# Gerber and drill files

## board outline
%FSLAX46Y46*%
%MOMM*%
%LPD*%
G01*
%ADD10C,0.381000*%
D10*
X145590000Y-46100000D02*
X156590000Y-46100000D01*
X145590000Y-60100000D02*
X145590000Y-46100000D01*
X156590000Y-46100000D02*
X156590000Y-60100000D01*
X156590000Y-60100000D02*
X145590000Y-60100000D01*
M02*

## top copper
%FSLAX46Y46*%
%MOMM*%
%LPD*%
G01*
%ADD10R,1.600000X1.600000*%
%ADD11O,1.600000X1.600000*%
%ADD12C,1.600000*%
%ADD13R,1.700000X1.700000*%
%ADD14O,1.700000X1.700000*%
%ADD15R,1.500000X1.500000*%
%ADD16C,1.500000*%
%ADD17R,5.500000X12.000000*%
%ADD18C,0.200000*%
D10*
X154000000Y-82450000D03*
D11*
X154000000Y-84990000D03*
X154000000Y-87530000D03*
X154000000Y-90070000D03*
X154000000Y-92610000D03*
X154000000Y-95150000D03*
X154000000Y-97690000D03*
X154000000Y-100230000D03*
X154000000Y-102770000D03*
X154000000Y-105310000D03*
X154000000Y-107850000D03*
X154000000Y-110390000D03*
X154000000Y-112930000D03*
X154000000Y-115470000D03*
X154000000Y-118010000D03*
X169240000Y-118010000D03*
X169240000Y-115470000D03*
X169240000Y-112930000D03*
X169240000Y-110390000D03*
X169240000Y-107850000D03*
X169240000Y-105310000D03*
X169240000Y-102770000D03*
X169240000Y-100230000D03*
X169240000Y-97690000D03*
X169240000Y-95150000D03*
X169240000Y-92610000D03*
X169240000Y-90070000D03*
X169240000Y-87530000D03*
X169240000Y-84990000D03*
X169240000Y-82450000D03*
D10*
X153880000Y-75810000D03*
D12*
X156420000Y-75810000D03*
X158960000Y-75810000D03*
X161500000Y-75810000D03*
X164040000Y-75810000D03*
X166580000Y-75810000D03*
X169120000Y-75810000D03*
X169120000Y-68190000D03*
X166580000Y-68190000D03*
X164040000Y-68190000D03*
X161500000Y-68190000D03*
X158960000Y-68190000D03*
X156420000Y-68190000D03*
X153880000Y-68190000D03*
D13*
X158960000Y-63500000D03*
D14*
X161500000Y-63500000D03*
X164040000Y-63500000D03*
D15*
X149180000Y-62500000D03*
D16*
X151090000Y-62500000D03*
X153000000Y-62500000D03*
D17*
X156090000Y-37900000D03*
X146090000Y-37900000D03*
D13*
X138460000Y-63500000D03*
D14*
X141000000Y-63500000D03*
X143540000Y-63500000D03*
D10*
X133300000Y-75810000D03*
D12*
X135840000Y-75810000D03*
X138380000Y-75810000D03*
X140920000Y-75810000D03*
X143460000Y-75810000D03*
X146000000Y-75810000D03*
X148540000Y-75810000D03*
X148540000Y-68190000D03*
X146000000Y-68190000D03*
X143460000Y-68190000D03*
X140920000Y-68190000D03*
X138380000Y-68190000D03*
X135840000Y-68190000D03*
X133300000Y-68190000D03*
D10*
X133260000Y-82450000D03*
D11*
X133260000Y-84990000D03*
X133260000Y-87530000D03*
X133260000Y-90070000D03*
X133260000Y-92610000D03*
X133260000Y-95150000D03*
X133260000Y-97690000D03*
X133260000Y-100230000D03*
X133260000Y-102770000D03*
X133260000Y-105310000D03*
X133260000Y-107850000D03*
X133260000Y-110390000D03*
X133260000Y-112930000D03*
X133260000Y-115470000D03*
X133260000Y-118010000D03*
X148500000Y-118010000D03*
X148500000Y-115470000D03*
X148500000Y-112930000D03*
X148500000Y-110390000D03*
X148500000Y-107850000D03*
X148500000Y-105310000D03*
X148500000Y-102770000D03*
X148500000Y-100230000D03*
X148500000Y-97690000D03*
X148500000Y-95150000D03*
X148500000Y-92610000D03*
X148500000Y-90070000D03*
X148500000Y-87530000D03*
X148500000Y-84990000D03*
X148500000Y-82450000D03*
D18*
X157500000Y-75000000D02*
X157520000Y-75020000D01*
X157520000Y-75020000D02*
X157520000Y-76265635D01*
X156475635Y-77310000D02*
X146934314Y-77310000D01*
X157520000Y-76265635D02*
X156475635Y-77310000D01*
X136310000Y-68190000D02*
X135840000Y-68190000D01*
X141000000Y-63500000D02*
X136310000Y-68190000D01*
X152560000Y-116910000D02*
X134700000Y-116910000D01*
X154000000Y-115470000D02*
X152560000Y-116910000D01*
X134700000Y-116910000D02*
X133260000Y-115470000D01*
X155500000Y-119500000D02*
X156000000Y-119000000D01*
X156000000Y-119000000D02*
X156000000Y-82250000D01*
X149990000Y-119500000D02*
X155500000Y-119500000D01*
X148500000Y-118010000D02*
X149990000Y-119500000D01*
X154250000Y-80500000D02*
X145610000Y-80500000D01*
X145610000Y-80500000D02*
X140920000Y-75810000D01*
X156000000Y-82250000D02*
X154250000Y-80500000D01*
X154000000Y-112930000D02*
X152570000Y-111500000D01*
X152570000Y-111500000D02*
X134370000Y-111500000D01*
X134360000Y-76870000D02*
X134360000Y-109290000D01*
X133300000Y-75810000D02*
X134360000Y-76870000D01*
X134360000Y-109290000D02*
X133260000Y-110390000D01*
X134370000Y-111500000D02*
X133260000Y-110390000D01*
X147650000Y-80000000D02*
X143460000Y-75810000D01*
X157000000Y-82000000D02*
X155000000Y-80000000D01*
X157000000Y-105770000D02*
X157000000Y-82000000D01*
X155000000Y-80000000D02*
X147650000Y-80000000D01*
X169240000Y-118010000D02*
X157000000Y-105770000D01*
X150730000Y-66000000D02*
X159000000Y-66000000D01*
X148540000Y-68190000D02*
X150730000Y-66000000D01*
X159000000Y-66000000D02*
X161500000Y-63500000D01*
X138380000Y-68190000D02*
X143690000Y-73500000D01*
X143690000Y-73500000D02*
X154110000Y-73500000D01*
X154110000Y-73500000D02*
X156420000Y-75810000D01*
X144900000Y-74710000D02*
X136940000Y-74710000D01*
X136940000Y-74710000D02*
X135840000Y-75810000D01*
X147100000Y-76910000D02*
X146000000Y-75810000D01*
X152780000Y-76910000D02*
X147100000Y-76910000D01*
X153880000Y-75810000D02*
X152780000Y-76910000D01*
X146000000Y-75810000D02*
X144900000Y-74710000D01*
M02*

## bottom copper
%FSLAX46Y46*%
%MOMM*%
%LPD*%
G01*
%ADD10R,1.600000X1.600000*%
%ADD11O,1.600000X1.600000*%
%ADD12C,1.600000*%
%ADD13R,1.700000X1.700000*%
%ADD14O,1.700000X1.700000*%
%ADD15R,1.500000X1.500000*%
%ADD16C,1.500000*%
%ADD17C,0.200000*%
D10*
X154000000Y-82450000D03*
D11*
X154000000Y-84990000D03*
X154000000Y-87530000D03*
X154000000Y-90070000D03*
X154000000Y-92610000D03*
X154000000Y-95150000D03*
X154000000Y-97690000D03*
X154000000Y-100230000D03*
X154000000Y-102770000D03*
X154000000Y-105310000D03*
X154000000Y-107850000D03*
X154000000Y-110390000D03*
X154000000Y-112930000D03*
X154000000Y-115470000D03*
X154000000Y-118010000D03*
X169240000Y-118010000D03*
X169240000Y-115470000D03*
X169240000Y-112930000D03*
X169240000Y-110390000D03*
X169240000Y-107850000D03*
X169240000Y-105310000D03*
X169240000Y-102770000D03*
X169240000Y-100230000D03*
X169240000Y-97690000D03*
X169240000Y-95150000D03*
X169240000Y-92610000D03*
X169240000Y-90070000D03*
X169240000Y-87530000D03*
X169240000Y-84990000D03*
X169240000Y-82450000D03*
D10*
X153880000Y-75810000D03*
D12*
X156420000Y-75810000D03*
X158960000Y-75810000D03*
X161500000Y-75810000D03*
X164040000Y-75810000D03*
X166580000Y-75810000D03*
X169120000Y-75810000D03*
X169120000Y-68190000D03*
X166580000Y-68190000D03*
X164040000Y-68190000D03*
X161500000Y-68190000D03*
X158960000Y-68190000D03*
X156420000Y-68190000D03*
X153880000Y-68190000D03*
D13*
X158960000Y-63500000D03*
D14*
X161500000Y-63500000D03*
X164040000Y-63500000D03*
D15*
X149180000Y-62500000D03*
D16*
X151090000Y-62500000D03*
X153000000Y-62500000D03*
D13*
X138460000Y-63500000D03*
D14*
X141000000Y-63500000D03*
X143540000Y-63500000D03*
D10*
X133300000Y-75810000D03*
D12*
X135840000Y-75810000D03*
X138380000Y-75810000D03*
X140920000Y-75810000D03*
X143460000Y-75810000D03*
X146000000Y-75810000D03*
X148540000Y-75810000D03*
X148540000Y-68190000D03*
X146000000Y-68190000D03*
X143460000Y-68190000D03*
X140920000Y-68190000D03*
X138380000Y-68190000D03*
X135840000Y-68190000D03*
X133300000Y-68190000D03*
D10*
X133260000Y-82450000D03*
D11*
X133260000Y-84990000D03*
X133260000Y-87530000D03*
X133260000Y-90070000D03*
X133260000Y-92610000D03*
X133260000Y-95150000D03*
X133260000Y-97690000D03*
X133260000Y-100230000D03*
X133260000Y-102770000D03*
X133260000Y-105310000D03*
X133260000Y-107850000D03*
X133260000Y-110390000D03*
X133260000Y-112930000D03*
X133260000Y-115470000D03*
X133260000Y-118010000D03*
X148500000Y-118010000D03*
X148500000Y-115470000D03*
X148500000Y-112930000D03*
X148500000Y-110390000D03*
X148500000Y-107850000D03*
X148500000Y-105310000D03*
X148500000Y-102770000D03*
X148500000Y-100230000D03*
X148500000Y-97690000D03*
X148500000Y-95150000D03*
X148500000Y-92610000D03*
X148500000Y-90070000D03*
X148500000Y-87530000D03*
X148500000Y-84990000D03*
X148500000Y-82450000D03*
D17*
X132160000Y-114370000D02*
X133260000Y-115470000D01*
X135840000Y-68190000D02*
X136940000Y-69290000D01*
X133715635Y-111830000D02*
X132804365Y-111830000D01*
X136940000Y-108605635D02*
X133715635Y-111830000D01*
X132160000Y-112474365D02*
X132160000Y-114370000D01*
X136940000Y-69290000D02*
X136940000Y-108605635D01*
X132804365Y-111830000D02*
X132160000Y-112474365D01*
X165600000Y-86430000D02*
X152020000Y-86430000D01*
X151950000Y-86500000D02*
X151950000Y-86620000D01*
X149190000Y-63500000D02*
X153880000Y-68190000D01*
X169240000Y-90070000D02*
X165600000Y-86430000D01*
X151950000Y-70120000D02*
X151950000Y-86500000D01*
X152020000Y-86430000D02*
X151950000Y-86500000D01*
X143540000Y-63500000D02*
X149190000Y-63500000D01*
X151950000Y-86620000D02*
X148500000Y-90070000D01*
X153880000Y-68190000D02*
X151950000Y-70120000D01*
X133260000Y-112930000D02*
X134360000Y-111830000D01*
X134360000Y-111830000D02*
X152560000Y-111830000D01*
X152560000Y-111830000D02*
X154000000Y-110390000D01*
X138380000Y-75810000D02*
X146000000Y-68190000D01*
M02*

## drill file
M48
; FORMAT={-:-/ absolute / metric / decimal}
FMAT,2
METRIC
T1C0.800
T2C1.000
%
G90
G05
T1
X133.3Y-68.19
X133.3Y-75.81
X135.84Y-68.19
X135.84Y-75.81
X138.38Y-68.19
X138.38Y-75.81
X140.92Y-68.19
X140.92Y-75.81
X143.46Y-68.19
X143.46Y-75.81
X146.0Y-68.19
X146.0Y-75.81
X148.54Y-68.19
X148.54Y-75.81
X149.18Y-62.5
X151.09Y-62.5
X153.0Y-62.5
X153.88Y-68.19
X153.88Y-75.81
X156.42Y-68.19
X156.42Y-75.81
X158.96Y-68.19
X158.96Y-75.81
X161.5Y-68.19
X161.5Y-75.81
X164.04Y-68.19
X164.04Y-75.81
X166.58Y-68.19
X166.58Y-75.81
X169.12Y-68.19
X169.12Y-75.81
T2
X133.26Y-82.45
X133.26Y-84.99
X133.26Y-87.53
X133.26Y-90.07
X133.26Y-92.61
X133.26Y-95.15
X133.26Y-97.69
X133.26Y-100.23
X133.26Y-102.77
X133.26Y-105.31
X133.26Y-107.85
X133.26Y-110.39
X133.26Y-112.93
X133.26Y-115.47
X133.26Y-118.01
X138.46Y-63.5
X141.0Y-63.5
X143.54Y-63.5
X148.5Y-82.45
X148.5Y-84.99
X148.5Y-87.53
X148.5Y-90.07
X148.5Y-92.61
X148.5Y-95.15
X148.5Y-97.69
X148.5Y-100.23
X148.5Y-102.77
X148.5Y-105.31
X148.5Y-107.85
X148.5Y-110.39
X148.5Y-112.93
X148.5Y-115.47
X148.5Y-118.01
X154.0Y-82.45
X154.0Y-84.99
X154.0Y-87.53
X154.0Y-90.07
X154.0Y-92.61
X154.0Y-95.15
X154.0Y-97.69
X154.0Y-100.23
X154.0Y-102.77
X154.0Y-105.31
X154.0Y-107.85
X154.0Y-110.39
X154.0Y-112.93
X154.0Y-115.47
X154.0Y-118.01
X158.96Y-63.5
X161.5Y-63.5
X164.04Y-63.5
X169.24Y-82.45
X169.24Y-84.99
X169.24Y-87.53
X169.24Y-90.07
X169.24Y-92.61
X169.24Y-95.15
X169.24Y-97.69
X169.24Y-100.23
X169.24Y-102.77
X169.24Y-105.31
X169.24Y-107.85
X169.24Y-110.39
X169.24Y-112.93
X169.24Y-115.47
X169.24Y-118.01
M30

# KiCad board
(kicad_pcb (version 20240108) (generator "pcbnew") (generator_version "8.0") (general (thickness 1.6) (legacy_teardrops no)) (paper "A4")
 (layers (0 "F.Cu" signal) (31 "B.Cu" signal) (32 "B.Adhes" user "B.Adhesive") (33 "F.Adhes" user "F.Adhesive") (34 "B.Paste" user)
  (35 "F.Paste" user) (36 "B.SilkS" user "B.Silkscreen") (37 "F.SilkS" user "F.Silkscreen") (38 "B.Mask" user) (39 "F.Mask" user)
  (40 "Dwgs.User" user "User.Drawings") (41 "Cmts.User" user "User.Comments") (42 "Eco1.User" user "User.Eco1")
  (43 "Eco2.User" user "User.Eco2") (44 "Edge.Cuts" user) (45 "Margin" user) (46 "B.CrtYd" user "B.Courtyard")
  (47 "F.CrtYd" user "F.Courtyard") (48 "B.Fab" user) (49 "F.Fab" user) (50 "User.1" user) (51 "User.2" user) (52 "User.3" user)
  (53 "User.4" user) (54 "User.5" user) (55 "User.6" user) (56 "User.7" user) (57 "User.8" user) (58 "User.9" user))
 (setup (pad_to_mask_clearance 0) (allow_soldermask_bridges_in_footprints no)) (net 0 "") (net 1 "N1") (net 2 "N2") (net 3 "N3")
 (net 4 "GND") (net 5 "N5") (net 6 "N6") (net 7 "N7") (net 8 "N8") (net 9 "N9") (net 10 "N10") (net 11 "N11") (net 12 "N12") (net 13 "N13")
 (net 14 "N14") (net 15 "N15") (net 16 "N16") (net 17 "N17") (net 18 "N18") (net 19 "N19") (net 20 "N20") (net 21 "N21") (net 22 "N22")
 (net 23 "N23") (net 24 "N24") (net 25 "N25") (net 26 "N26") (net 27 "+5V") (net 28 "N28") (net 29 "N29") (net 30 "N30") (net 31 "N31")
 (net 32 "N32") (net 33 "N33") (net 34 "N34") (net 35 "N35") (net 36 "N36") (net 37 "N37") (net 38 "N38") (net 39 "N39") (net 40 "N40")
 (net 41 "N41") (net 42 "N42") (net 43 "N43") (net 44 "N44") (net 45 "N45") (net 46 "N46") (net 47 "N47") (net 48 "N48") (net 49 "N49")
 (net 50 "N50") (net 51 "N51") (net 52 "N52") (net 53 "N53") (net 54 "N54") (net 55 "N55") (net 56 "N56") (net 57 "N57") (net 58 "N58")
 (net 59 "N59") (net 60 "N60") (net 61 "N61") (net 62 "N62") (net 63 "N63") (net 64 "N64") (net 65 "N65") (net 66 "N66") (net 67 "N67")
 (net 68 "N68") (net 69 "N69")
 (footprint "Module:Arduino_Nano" (layer "F.Cu") (at 154 82.45)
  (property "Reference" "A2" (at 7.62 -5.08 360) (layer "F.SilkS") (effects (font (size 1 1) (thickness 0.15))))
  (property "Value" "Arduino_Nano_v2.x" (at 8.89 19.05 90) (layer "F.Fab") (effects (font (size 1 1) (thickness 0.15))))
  (pad "1" thru_hole rect (at 0 0) (size 1.6 1.6) (drill 1) (layers "*.Cu" "*.Mask") (remove_unused_layers no) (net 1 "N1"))
  (pad "2" thru_hole oval (at 0 2.54) (size 1.6 1.6) (drill 1) (layers "*.Cu" "*.Mask") (remove_unused_layers no) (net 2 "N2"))
  (pad "3" thru_hole oval (at 0 5.08) (size 1.6 1.6) (drill 1) (layers "*.Cu" "*.Mask") (remove_unused_layers no) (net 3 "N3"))
  (pad "4" thru_hole oval (at 0 7.62) (size 1.6 1.6) (drill 1) (layers "*.Cu" "*.Mask") (remove_unused_layers no) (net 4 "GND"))
  (pad "5" thru_hole oval (at 0 10.16) (size 1.6 1.6) (drill 1) (layers "*.Cu" "*.Mask") (remove_unused_layers no) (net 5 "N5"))
  (pad "6" thru_hole oval (at 0 12.7) (size 1.6 1.6) (drill 1) (layers "*.Cu" "*.Mask") (remove_unused_layers no) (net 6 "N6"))
  (pad "7" thru_hole oval (at 0 15.24) (size 1.6 1.6) (drill 1) (layers "*.Cu" "*.Mask") (remove_unused_layers no) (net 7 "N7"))
  (pad "8" thru_hole oval (at 0 17.78) (size 1.6 1.6) (drill 1) (layers "*.Cu" "*.Mask") (remove_unused_layers no) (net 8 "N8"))
  (pad "9" thru_hole oval (at 0 20.32) (size 1.6 1.6) (drill 1) (layers "*.Cu" "*.Mask") (remove_unused_layers no) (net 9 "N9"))
  (pad "10" thru_hole oval (at 0 22.86) (size 1.6 1.6) (drill 1) (layers "*.Cu" "*.Mask") (remove_unused_layers no) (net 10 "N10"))
  (pad "11" thru_hole oval (at 0 25.4) (size 1.6 1.6) (drill 1) (layers "*.Cu" "*.Mask") (remove_unused_layers no) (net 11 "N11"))
  (pad "12" thru_hole oval (at 0 27.94) (size 1.6 1.6) (drill 1) (layers "*.Cu" "*.Mask") (remove_unused_layers no) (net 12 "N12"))
  (pad "13" thru_hole oval (at 0 30.48) (size 1.6 1.6) (drill 1) (layers "*.Cu" "*.Mask") (remove_unused_layers no) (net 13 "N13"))
  (pad "14" thru_hole oval (at 0 33.02) (size 1.6 1.6) (drill 1) (layers "*.Cu" "*.Mask") (remove_unused_layers no) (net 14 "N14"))
  (pad "15" thru_hole oval (at 0 35.56) (size 1.6 1.6) (drill 1) (layers "*.Cu" "*.Mask") (remove_unused_layers no) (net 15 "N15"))
  (pad "16" thru_hole oval (at 15.24 35.56) (size 1.6 1.6) (drill 1) (layers "*.Cu" "*.Mask") (remove_unused_layers no) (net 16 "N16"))
  (pad "17" thru_hole oval (at 15.24 33.02) (size 1.6 1.6) (drill 1) (layers "*.Cu" "*.Mask") (remove_unused_layers no) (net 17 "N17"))
  (pad "18" thru_hole oval (at 15.24 30.48) (size 1.6 1.6) (drill 1) (layers "*.Cu" "*.Mask") (remove_unused_layers no) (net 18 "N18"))
  (pad "19" thru_hole oval (at 15.24 27.94) (size 1.6 1.6) (drill 1) (layers "*.Cu" "*.Mask") (remove_unused_layers no) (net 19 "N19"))
  (pad "20" thru_hole oval (at 15.24 25.4) (size 1.6 1.6) (drill 1) (layers "*.Cu" "*.Mask") (remove_unused_layers no) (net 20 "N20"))
  (pad "21" thru_hole oval (at 15.24 22.86) (size 1.6 1.6) (drill 1) (layers "*.Cu" "*.Mask") (remove_unused_layers no) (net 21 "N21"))
  (pad "22" thru_hole oval (at 15.24 20.32) (size 1.6 1.6) (drill 1) (layers "*.Cu" "*.Mask") (remove_unused_layers no) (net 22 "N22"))
  (pad "23" thru_hole oval (at 15.24 17.78) (size 1.6 1.6) (drill 1) (layers "*.Cu" "*.Mask") (remove_unused_layers no) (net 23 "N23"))
  (pad "24" thru_hole oval (at 15.24 15.24) (size 1.6 1.6) (drill 1) (layers "*.Cu" "*.Mask") (remove_unused_layers no) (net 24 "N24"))
  (pad "25" thru_hole oval (at 15.24 12.7) (size 1.6 1.6) (drill 1) (layers "*.Cu" "*.Mask") (remove_unused_layers no) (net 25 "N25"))
  (pad "26" thru_hole oval (at 15.24 10.16) (size 1.6 1.6) (drill 1) (layers "*.Cu" "*.Mask") (remove_unused_layers no) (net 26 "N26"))
  (pad "27" thru_hole oval (at 15.24 7.62) (size 1.6 1.6) (drill 1) (layers "*.Cu" "*.Mask") (remove_unused_layers no) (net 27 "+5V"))
  (pad "28" thru_hole oval (at 15.24 5.08) (size 1.6 1.6) (drill 1) (layers "*.Cu" "*.Mask") (remove_unused_layers no) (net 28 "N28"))
  (pad "29" thru_hole oval (at 15.24 2.54) (size 1.6 1.6) (drill 1) (layers "*.Cu" "*.Mask") (remove_unused_layers no) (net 4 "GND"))
  (pad "30" thru_hole oval (at 15.24 0) (size 1.6 1.6) (drill 1) (layers "*.Cu" "*.Mask") (remove_unused_layers no) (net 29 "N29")))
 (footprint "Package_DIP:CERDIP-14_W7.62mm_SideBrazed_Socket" (layer "F.Cu") (at 153.88 75.81 90)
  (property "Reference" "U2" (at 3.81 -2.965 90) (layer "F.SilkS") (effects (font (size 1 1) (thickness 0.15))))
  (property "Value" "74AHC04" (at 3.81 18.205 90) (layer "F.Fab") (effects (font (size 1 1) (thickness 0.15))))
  (pad "1" thru_hole rect (at 0 0 90) (size 1.6 1.6) (drill 0.8) (layers "*.Cu" "*.Mask") (remove_unused_layers no) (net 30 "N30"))
  (pad "2" thru_hole circle (at 0 2.54 90) (size 1.6 1.6) (drill 0.8) (layers "*.Cu" "*.Mask") (remove_unused_layers no) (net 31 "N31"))
  (pad "3" thru_hole circle (at 0 5.08 90) (size 1.6 1.6) (drill 0.8) (layers "*.Cu" "*.Mask") (remove_unused_layers no) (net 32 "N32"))
  (pad "4" thru_hole circle (at 0 7.62 90) (size 1.6 1.6) (drill 0.8) (layers "*.Cu" "*.Mask") (remove_unused_layers no) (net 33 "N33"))
  (pad "5" thru_hole circle (at 0 10.16 90) (size 1.6 1.6) (drill 0.8) (layers "*.Cu" "*.Mask") (remove_unused_layers no) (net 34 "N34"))
  (pad "6" thru_hole circle (at 0 12.7 90) (size 1.6 1.6) (drill 0.8) (layers "*.Cu" "*.Mask") (remove_unused_layers no) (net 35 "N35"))
  (pad "7" thru_hole circle (at 0 15.24 90) (size 1.6 1.6) (drill 0.8) (layers "*.Cu" "*.Mask") (remove_unused_layers no) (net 4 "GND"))
  (pad "8" thru_hole circle (at 7.62 15.24 90) (size 1.6 1.6) (drill 0.8) (layers "*.Cu" "*.Mask") (remove_unused_layers no) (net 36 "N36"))
  (pad "9" thru_hole circle (at 7.62 12.7 90) (size 1.6 1.6) (drill 0.8) (layers "*.Cu" "*.Mask") (remove_unused_layers no) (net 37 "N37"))
  (pad "10" thru_hole circle (at 7.62 10.16 90) (size 1.6 1.6) (drill 0.8) (layers "*.Cu" "*.Mask") (remove_unused_layers no) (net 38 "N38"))
  (pad "11" thru_hole circle (at 7.62 7.62 90) (size 1.6 1.6) (drill 0.8) (layers "*.Cu" "*.Mask") (remove_unused_layers no) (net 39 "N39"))
  (pad "12" thru_hole circle (at 7.62 5.08 90) (size 1.6 1.6) (drill 0.8) (layers "*.Cu" "*.Mask") (remove_unused_layers no) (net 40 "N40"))
  (pad "13" thru_hole circle (at 7.62 2.54 90) (size 1.6 1.6) (drill 0.8) (layers "*.Cu" "*.Mask") (remove_unused_layers no) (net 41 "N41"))
  (pad "14" thru_hole circle (at 7.62 0 90) (size 1.6 1.6) (drill 0.8) (layers "*.Cu" "*.Mask") (remove_unused_layers no) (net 27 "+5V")))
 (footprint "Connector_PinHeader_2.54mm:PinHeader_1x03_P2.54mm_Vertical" (layer "F.Cu") (at 158.96 63.5 90)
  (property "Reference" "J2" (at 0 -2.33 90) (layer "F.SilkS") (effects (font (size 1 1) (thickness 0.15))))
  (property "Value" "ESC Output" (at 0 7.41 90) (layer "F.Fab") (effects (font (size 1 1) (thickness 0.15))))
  (pad "1" thru_hole rect (at 0 0 90) (size 1.7 1.7) (drill 1) (layers "*.Cu" "*.Mask") (remove_unused_layers no) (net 4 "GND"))
  (pad "2" thru_hole oval (at 0 2.54 90) (size 1.7 1.7) (drill 1) (layers "*.Cu" "*.Mask") (remove_unused_layers no) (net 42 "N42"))
  (pad "3" thru_hole oval (at 0 5.08 90) (size 1.7 1.7) (drill 1) (layers "*.Cu" "*.Mask") (remove_unused_layers no) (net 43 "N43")))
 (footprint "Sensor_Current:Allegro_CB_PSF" (layer "F.Cu") (at 149.18 62.5)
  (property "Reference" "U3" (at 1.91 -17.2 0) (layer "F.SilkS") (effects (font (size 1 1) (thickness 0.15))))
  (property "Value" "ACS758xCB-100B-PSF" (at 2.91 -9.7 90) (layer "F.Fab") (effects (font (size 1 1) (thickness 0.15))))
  (fp_line (start -3.59 -16.4) (end 7.41 -16.4) (stroke (width 0.381) (type solid)) (layer "Edge.Cuts"))
  (fp_line (start -3.59 -2.4) (end -3.59 -16.4) (stroke (width 0.381) (type solid)) (layer "Edge.Cuts"))
  (fp_line (start 7.41 -16.4) (end 7.41 -2.4) (stroke (width 0.381) (type solid)) (layer "Edge.Cuts"))
  (fp_line (start 7.41 -2.4) (end -3.59 -2.4) (stroke (width 0.381) (type solid)) (layer "Edge.Cuts"))
  (pad "1" thru_hole rect (at 0 0) (size 1.5 1.5) (drill 0.8) (layers "*.Cu" "*.Mask") (remove_unused_layers no) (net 27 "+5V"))
  (pad "2" thru_hole circle (at 1.91 0) (size 1.5 1.5) (drill 0.8) (layers "*.Cu" "*.Mask") (remove_unused_layers no) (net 4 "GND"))
  (pad "3" thru_hole circle (at 3.82 0) (size 1.5 1.5) (drill 0.8) (layers "*.Cu" "*.Mask") (remove_unused_layers no) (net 19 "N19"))
  (pad "4" smd rect (at 6.91 -24.6) (size 5.5 12) (layers "F.Cu" "F.Paste" "F.Mask") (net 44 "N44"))
  (pad "5" smd rect (at -3.09 -24.6) (size 5.5 12) (layers "F.Cu" "F.Paste" "F.Mask") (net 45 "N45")))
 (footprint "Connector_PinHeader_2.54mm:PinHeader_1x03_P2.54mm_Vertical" (layer "F.Cu") (at 138.46 63.5 90)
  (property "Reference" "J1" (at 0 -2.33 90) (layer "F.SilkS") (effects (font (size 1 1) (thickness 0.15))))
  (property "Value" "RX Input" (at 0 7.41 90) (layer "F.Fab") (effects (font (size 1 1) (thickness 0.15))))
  (pad "1" thru_hole rect (at 0 0 90) (size 1.7 1.7) (drill 1) (layers "*.Cu" "*.Mask") (remove_unused_layers no) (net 4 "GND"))
  (pad "2" thru_hole oval (at 0 2.54 90) (size 1.7 1.7) (drill 1) (layers "*.Cu" "*.Mask") (remove_unused_layers no) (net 14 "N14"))
  (pad "3" thru_hole oval (at 0 5.08 90) (size 1.7 1.7) (drill 1) (layers "*.Cu" "*.Mask") (remove_unused_layers no) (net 27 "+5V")))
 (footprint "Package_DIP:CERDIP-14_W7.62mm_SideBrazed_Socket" (layer "F.Cu") (at 133.3 75.81 90)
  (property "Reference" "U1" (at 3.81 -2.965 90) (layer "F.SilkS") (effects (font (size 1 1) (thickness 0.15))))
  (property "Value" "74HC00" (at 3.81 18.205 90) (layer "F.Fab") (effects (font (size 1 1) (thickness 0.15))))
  (pad "1" thru_hole rect (at 0 0 90) (size 1.6 1.6) (drill 0.8) (layers "*.Cu" "*.Mask") (remove_unused_layers no) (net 13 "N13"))
  (pad "2" thru_hole circle (at 0 2.54 90) (size 1.6 1.6) (drill 0.8) (layers "*.Cu" "*.Mask") (remove_unused_layers no) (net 30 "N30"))
  (pad "3" thru_hole circle (at 0 5.08 90) (size 1.6 1.6) (drill 0.8) (layers "*.Cu" "*.Mask") (remove_unused_layers no) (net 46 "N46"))
  (pad "4" thru_hole circle (at 0 7.62 90) (size 1.6 1.6) (drill 0.8) (layers "*.Cu" "*.Mask") (remove_unused_layers no) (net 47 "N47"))
  (pad "5" thru_hole circle (at 0 10.16 90) (size 1.6 1.6) (drill 0.8) (layers "*.Cu" "*.Mask") (remove_unused_layers no) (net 16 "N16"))
  (pad "6" thru_hole circle (at 0 12.7 90) (size 1.6 1.6) (drill 0.8) (layers "*.Cu" "*.Mask") (remove_unused_layers no) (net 30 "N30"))
  (pad "7" thru_hole circle (at 0 15.24 90) (size 1.6 1.6) (drill 0.8) (layers "*.Cu" "*.Mask") (remove_unused_layers no) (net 4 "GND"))
  (pad "8" thru_hole circle (at 7.62 15.24 90) (size 1.6 1.6) (drill 0.8) (layers "*.Cu" "*.Mask") (remove_unused_layers no) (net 42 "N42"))
  (pad "9" thru_hole circle (at 7.62 12.7 90) (size 1.6 1.6) (drill 0.8) (layers "*.Cu" "*.Mask") (remove_unused_layers no) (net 46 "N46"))
  (pad "10" thru_hole circle (at 7.62 10.16 90) (size 1.6 1.6) (drill 0.8) (layers "*.Cu" "*.Mask") (remove_unused_layers no) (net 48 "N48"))
  (pad "11" thru_hole circle (at 7.62 7.62 90) (size 1.6 1.6) (drill 0.8) (layers "*.Cu" "*.Mask") (remove_unused_layers no) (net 48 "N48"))
  (pad "12" thru_hole circle (at 7.62 5.08 90) (size 1.6 1.6) (drill 0.8) (layers "*.Cu" "*.Mask") (remove_unused_layers no) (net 31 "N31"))
  (pad "13" thru_hole circle (at 7.62 2.54 90) (size 1.6 1.6) (drill 0.8) (layers "*.Cu" "*.Mask") (remove_unused_layers no) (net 14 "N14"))
  (pad "14" thru_hole circle (at 7.62 0 90) (size 1.6 1.6) (drill 0.8) (layers "*.Cu" "*.Mask") (remove_unused_layers no) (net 27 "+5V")))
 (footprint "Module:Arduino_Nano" (layer "F.Cu") (at 133.26 82.45)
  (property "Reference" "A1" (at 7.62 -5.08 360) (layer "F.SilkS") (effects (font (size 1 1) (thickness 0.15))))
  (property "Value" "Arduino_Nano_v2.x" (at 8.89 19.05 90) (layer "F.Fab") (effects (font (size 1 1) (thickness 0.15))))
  (pad "1" thru_hole rect (at 0 0) (size 1.6 1.6) (drill 1) (layers "*.Cu" "*.Mask") (remove_unused_layers no) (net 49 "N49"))
  (pad "2" thru_hole oval (at 0 2.54) (size 1.6 1.6) (drill 1) (layers "*.Cu" "*.Mask") (remove_unused_layers no) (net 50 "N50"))
  (pad "3" thru_hole oval (at 0 5.08) (size 1.6 1.6) (drill 1) (layers "*.Cu" "*.Mask") (remove_unused_layers no) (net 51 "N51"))
  (pad "4" thru_hole oval (at 0 7.62) (size 1.6 1.6) (drill 1) (layers "*.Cu" "*.Mask") (remove_unused_layers no) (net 4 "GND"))
  (pad "5" thru_hole oval (at 0 10.16) (size 1.6 1.6) (drill 1) (layers "*.Cu" "*.Mask") (remove_unused_layers no) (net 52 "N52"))
  (pad "6" thru_hole oval (at 0 12.7) (size 1.6 1.6) (drill 1) (layers "*.Cu" "*.Mask") (remove_unused_layers no) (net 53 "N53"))
  (pad "7" thru_hole oval (at 0 15.24) (size 1.6 1.6) (drill 1) (layers "*.Cu" "*.Mask") (remove_unused_layers no) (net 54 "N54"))
  (pad "8" thru_hole oval (at 0 17.78) (size 1.6 1.6) (drill 1) (layers "*.Cu" "*.Mask") (remove_unused_layers no) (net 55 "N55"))
  (pad "9" thru_hole oval (at 0 20.32) (size 1.6 1.6) (drill 1) (layers "*.Cu" "*.Mask") (remove_unused_layers no) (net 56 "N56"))
  (pad "10" thru_hole oval (at 0 22.86) (size 1.6 1.6) (drill 1) (layers "*.Cu" "*.Mask") (remove_unused_layers no) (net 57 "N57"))
  (pad "11" thru_hole oval (at 0 25.4) (size 1.6 1.6) (drill 1) (layers "*.Cu" "*.Mask") (remove_unused_layers no) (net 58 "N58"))
  (pad "12" thru_hole oval (at 0 27.94) (size 1.6 1.6) (drill 1) (layers "*.Cu" "*.Mask") (remove_unused_layers no) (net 13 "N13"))
  (pad "13" thru_hole oval (at 0 30.48) (size 1.6 1.6) (drill 1) (layers "*.Cu" "*.Mask") (remove_unused_layers no) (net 12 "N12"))
  (pad "14" thru_hole oval (at 0 33.02) (size 1.6 1.6) (drill 1) (layers "*.Cu" "*.Mask") (remove_unused_layers no) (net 14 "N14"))
  (pad "15" thru_hole oval (at 0 35.56) (size 1.6 1.6) (drill 1) (layers "*.Cu" "*.Mask") (remove_unused_layers no) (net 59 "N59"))
  (pad "16" thru_hole oval (at 15.24 35.56) (size 1.6 1.6) (drill 1) (layers "*.Cu" "*.Mask") (remove_unused_layers no) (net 47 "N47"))
  (pad "17" thru_hole oval (at 15.24 33.02) (size 1.6 1.6) (drill 1) (layers "*.Cu" "*.Mask") (remove_unused_layers no) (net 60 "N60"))
  (pad "18" thru_hole oval (at 15.24 30.48) (size 1.6 1.6) (drill 1) (layers "*.Cu" "*.Mask") (remove_unused_layers no) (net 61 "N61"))
  (pad "19" thru_hole oval (at 15.24 27.94) (size 1.6 1.6) (drill 1) (layers "*.Cu" "*.Mask") (remove_unused_layers no) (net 19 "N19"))
  (pad "20" thru_hole oval (at 15.24 25.4) (size 1.6 1.6) (drill 1) (layers "*.Cu" "*.Mask") (remove_unused_layers no) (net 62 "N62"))
  (pad "21" thru_hole oval (at 15.24 22.86) (size 1.6 1.6) (drill 1) (layers "*.Cu" "*.Mask") (remove_unused_layers no) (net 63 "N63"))
  (pad "22" thru_hole oval (at 15.24 20.32) (size 1.6 1.6) (drill 1) (layers "*.Cu" "*.Mask") (remove_unused_layers no) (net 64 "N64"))
  (pad "23" thru_hole oval (at 15.24 17.78) (size 1.6 1.6) (drill 1) (layers "*.Cu" "*.Mask") (remove_unused_layers no) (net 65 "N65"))
  (pad "24" thru_hole oval (at 15.24 15.24) (size 1.6 1.6) (drill 1) (layers "*.Cu" "*.Mask") (remove_unused_layers no) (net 24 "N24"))
  (pad "25" thru_hole oval (at 15.24 12.7) (size 1.6 1.6) (drill 1) (layers "*.Cu" "*.Mask") (remove_unused_layers no) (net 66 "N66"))
  (pad "26" thru_hole oval (at 15.24 10.16) (size 1.6 1.6) (drill 1) (layers "*.Cu" "*.Mask") (remove_unused_layers no) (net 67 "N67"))
  (pad "27" thru_hole oval (at 15.24 7.62) (size 1.6 1.6) (drill 1) (layers "*.Cu" "*.Mask") (remove_unused_layers no) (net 27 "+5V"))
  (pad "28" thru_hole oval (at 15.24 5.08) (size 1.6 1.6) (drill 1) (layers "*.Cu" "*.Mask") (remove_unused_layers no) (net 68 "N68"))
  (pad "29" thru_hole oval (at 15.24 2.54) (size 1.6 1.6) (drill 1) (layers "*.Cu" "*.Mask") (remove_unused_layers no) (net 4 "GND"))
  (pad "30" thru_hole oval (at 15.24 0) (size 1.6 1.6) (drill 1) (layers "*.Cu" "*.Mask") (remove_unused_layers no) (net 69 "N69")))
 (segment (start 157.5 75) (end 157.52 75.02) (width 0.2) (layer "F.Cu") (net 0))
 (segment (start 157.52 75.02) (end 157.52 76.265635) (width 0.2) (layer "F.Cu") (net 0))
 (segment (start 156.475635 77.31) (end 146.934314 77.31) (width 0.2) (layer "F.Cu") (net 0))
 (segment (start 157.52 76.265635) (end 156.475635 77.31) (width 0.2) (layer "F.Cu") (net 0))
 (segment (start 136.31 68.19) (end 135.84 68.19) (width 0.2) (layer "F.Cu") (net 14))
 (segment (start 141 63.5) (end 136.31 68.19) (width 0.2) (layer "F.Cu") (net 14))
 (segment (start 152.56 116.91) (end 134.7 116.91) (width 0.2) (layer "F.Cu") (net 14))
 (segment (start 154 115.47) (end 152.56 116.91) (width 0.2) (layer "F.Cu") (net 14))
 (segment (start 134.7 116.91) (end 133.26 115.47) (width 0.2) (layer "F.Cu") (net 14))
 (segment (start 132.16 114.37) (end 133.26 115.47) (width 0.2) (layer "B.Cu") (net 14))
 (segment (start 135.84 68.19) (end 136.94 69.29) (width 0.2) (layer "B.Cu") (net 14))
 (segment (start 133.715635 111.83) (end 132.804365 111.83) (width 0.2) (layer "B.Cu") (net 14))
 (segment (start 136.94 108.605635) (end 133.715635 111.83) (width 0.2) (layer "B.Cu") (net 14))
 (segment (start 132.16 112.474365) (end 132.16 114.37) (width 0.2) (layer "B.Cu") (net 14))
 (segment (start 136.94 69.29) (end 136.94 108.605635) (width 0.2) (layer "B.Cu") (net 14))
 (segment (start 132.804365 111.83) (end 132.16 112.474365) (width 0.2) (layer "B.Cu") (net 14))
 (segment (start 165.6 86.43) (end 152.02 86.43) (width 0.2) (layer "B.Cu") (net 27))
 (segment (start 151.95 86.5) (end 151.95 86.62) (width 0.2) (layer "B.Cu") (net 27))
 (segment (start 149.19 63.5) (end 153.88 68.19) (width 0.2) (layer "B.Cu") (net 27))
 (segment (start 169.24 90.07) (end 165.6 86.43) (width 0.2) (layer "B.Cu") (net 27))
 (segment (start 151.95 70.12) (end 151.95 86.5) (width 0.2) (layer "B.Cu") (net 27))
 (segment (start 152.02 86.43) (end 151.95 86.5) (width 0.2) (layer "B.Cu") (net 27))
 (segment (start 143.54 63.5) (end 149.19 63.5) (width 0.2) (layer "B.Cu") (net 27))
 (segment (start 151.95 86.62) (end 148.5 90.07) (width 0.2) (layer "B.Cu") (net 27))
 (segment (start 153.88 68.19) (end 151.95 70.12) (width 0.2) (layer "B.Cu") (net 27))
 (segment (start 155.5 119.5) (end 156 119) (width 0.2) (layer "F.Cu") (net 47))
 (segment (start 156 119) (end 156 82.25) (width 0.2) (layer "F.Cu") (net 47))
 (segment (start 149.99 119.5) (end 155.5 119.5) (width 0.2) (layer "F.Cu") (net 47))
 (segment (start 148.5 118.01) (end 149.99 119.5) (width 0.2) (layer "F.Cu") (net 47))
 (segment (start 154.25 80.5) (end 145.61 80.5) (width 0.2) (layer "F.Cu") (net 47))
 (segment (start 145.61 80.5) (end 140.92 75.81) (width 0.2) (layer "F.Cu") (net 47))
 (segment (start 156 82.25) (end 154.25 80.5) (width 0.2) (layer "F.Cu") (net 47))
 (segment (start 154 112.93) (end 152.57 111.5) (width 0.2) (layer "F.Cu") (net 13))
 (segment (start 152.57 111.5) (end 134.37 111.5) (width 0.2) (layer "F.Cu") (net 13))
 (segment (start 134.36 76.87) (end 134.36 109.29) (width 0.2) (layer "F.Cu") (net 13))
 (segment (start 133.3 75.81) (end 134.36 76.87) (width 0.2) (layer "F.Cu") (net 13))
 (segment (start 134.36 109.29) (end 133.26 110.39) (width 0.2) (layer "F.Cu") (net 13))
 (segment (start 134.37 111.5) (end 133.26 110.39) (width 0.2) (layer "F.Cu") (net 13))
 (segment (start 133.26 112.93) (end 134.36 111.83) (width 0.2) (layer "B.Cu") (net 12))
 (segment (start 134.36 111.83) (end 152.56 111.83) (width 0.2) (layer "B.Cu") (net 12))
 (segment (start 152.56 111.83) (end 154 110.39) (width 0.2) (layer "B.Cu") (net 12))
 (segment (start 147.65 80) (end 143.46 75.81) (width 0.2) (layer "F.Cu") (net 16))
 (segment (start 157 82) (end 155 80) (width 0.2) (layer "F.Cu") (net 16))
 (segment (start 157 105.77) (end 157 82) (width 0.2) (layer "F.Cu") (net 16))
 (segment (start 155 80) (end 147.65 80) (width 0.2) (layer "F.Cu") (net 16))
 (segment (start 169.24 118.01) (end 157 105.77) (width 0.2) (layer "F.Cu") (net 16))
 (segment (start 150.73 66) (end 159 66) (width 0.2) (layer "F.Cu") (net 42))
 (segment (start 148.54 68.19) (end 150.73 66) (width 0.2) (layer "F.Cu") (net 42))
 (segment (start 159 66) (end 161.5 63.5) (width 0.2) (layer "F.Cu") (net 42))
 (segment (start 138.38 75.81) (end 146 68.19) (width 0.2) (layer "B.Cu") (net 46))
 (segment (start 138.38 68.19) (end 143.69 73.5) (width 0.2) (layer "F.Cu") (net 31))
 (segment (start 143.69 73.5) (end 154.11 73.5) (width 0.2) (layer "F.Cu") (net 31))
 (segment (start 154.11 73.5) (end 156.42 75.81) (width 0.2) (layer "F.Cu") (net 31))
 (segment (start 144.9 74.71) (end 136.94 74.71) (width 0.2) (layer "F.Cu") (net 30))
 (segment (start 136.94 74.71) (end 135.84 75.81) (width 0.2) (layer "F.Cu") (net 30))
 (segment (start 147.1 76.91) (end 146 75.81) (width 0.2) (layer "F.Cu") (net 30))
 (segment (start 152.78 76.91) (end 147.1 76.91) (width 0.2) (layer "F.Cu") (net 30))
 (segment (start 153.88 75.81) (end 152.78 76.91) (width 0.2) (layer "F.Cu") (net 30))
 (segment (start 146 75.81) (end 144.9 74.71) (width 0.2) (layer "F.Cu") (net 30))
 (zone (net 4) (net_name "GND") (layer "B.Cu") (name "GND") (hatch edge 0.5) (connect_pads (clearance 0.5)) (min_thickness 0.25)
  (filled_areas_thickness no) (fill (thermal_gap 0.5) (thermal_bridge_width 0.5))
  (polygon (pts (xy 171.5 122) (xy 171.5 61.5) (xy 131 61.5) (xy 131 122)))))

